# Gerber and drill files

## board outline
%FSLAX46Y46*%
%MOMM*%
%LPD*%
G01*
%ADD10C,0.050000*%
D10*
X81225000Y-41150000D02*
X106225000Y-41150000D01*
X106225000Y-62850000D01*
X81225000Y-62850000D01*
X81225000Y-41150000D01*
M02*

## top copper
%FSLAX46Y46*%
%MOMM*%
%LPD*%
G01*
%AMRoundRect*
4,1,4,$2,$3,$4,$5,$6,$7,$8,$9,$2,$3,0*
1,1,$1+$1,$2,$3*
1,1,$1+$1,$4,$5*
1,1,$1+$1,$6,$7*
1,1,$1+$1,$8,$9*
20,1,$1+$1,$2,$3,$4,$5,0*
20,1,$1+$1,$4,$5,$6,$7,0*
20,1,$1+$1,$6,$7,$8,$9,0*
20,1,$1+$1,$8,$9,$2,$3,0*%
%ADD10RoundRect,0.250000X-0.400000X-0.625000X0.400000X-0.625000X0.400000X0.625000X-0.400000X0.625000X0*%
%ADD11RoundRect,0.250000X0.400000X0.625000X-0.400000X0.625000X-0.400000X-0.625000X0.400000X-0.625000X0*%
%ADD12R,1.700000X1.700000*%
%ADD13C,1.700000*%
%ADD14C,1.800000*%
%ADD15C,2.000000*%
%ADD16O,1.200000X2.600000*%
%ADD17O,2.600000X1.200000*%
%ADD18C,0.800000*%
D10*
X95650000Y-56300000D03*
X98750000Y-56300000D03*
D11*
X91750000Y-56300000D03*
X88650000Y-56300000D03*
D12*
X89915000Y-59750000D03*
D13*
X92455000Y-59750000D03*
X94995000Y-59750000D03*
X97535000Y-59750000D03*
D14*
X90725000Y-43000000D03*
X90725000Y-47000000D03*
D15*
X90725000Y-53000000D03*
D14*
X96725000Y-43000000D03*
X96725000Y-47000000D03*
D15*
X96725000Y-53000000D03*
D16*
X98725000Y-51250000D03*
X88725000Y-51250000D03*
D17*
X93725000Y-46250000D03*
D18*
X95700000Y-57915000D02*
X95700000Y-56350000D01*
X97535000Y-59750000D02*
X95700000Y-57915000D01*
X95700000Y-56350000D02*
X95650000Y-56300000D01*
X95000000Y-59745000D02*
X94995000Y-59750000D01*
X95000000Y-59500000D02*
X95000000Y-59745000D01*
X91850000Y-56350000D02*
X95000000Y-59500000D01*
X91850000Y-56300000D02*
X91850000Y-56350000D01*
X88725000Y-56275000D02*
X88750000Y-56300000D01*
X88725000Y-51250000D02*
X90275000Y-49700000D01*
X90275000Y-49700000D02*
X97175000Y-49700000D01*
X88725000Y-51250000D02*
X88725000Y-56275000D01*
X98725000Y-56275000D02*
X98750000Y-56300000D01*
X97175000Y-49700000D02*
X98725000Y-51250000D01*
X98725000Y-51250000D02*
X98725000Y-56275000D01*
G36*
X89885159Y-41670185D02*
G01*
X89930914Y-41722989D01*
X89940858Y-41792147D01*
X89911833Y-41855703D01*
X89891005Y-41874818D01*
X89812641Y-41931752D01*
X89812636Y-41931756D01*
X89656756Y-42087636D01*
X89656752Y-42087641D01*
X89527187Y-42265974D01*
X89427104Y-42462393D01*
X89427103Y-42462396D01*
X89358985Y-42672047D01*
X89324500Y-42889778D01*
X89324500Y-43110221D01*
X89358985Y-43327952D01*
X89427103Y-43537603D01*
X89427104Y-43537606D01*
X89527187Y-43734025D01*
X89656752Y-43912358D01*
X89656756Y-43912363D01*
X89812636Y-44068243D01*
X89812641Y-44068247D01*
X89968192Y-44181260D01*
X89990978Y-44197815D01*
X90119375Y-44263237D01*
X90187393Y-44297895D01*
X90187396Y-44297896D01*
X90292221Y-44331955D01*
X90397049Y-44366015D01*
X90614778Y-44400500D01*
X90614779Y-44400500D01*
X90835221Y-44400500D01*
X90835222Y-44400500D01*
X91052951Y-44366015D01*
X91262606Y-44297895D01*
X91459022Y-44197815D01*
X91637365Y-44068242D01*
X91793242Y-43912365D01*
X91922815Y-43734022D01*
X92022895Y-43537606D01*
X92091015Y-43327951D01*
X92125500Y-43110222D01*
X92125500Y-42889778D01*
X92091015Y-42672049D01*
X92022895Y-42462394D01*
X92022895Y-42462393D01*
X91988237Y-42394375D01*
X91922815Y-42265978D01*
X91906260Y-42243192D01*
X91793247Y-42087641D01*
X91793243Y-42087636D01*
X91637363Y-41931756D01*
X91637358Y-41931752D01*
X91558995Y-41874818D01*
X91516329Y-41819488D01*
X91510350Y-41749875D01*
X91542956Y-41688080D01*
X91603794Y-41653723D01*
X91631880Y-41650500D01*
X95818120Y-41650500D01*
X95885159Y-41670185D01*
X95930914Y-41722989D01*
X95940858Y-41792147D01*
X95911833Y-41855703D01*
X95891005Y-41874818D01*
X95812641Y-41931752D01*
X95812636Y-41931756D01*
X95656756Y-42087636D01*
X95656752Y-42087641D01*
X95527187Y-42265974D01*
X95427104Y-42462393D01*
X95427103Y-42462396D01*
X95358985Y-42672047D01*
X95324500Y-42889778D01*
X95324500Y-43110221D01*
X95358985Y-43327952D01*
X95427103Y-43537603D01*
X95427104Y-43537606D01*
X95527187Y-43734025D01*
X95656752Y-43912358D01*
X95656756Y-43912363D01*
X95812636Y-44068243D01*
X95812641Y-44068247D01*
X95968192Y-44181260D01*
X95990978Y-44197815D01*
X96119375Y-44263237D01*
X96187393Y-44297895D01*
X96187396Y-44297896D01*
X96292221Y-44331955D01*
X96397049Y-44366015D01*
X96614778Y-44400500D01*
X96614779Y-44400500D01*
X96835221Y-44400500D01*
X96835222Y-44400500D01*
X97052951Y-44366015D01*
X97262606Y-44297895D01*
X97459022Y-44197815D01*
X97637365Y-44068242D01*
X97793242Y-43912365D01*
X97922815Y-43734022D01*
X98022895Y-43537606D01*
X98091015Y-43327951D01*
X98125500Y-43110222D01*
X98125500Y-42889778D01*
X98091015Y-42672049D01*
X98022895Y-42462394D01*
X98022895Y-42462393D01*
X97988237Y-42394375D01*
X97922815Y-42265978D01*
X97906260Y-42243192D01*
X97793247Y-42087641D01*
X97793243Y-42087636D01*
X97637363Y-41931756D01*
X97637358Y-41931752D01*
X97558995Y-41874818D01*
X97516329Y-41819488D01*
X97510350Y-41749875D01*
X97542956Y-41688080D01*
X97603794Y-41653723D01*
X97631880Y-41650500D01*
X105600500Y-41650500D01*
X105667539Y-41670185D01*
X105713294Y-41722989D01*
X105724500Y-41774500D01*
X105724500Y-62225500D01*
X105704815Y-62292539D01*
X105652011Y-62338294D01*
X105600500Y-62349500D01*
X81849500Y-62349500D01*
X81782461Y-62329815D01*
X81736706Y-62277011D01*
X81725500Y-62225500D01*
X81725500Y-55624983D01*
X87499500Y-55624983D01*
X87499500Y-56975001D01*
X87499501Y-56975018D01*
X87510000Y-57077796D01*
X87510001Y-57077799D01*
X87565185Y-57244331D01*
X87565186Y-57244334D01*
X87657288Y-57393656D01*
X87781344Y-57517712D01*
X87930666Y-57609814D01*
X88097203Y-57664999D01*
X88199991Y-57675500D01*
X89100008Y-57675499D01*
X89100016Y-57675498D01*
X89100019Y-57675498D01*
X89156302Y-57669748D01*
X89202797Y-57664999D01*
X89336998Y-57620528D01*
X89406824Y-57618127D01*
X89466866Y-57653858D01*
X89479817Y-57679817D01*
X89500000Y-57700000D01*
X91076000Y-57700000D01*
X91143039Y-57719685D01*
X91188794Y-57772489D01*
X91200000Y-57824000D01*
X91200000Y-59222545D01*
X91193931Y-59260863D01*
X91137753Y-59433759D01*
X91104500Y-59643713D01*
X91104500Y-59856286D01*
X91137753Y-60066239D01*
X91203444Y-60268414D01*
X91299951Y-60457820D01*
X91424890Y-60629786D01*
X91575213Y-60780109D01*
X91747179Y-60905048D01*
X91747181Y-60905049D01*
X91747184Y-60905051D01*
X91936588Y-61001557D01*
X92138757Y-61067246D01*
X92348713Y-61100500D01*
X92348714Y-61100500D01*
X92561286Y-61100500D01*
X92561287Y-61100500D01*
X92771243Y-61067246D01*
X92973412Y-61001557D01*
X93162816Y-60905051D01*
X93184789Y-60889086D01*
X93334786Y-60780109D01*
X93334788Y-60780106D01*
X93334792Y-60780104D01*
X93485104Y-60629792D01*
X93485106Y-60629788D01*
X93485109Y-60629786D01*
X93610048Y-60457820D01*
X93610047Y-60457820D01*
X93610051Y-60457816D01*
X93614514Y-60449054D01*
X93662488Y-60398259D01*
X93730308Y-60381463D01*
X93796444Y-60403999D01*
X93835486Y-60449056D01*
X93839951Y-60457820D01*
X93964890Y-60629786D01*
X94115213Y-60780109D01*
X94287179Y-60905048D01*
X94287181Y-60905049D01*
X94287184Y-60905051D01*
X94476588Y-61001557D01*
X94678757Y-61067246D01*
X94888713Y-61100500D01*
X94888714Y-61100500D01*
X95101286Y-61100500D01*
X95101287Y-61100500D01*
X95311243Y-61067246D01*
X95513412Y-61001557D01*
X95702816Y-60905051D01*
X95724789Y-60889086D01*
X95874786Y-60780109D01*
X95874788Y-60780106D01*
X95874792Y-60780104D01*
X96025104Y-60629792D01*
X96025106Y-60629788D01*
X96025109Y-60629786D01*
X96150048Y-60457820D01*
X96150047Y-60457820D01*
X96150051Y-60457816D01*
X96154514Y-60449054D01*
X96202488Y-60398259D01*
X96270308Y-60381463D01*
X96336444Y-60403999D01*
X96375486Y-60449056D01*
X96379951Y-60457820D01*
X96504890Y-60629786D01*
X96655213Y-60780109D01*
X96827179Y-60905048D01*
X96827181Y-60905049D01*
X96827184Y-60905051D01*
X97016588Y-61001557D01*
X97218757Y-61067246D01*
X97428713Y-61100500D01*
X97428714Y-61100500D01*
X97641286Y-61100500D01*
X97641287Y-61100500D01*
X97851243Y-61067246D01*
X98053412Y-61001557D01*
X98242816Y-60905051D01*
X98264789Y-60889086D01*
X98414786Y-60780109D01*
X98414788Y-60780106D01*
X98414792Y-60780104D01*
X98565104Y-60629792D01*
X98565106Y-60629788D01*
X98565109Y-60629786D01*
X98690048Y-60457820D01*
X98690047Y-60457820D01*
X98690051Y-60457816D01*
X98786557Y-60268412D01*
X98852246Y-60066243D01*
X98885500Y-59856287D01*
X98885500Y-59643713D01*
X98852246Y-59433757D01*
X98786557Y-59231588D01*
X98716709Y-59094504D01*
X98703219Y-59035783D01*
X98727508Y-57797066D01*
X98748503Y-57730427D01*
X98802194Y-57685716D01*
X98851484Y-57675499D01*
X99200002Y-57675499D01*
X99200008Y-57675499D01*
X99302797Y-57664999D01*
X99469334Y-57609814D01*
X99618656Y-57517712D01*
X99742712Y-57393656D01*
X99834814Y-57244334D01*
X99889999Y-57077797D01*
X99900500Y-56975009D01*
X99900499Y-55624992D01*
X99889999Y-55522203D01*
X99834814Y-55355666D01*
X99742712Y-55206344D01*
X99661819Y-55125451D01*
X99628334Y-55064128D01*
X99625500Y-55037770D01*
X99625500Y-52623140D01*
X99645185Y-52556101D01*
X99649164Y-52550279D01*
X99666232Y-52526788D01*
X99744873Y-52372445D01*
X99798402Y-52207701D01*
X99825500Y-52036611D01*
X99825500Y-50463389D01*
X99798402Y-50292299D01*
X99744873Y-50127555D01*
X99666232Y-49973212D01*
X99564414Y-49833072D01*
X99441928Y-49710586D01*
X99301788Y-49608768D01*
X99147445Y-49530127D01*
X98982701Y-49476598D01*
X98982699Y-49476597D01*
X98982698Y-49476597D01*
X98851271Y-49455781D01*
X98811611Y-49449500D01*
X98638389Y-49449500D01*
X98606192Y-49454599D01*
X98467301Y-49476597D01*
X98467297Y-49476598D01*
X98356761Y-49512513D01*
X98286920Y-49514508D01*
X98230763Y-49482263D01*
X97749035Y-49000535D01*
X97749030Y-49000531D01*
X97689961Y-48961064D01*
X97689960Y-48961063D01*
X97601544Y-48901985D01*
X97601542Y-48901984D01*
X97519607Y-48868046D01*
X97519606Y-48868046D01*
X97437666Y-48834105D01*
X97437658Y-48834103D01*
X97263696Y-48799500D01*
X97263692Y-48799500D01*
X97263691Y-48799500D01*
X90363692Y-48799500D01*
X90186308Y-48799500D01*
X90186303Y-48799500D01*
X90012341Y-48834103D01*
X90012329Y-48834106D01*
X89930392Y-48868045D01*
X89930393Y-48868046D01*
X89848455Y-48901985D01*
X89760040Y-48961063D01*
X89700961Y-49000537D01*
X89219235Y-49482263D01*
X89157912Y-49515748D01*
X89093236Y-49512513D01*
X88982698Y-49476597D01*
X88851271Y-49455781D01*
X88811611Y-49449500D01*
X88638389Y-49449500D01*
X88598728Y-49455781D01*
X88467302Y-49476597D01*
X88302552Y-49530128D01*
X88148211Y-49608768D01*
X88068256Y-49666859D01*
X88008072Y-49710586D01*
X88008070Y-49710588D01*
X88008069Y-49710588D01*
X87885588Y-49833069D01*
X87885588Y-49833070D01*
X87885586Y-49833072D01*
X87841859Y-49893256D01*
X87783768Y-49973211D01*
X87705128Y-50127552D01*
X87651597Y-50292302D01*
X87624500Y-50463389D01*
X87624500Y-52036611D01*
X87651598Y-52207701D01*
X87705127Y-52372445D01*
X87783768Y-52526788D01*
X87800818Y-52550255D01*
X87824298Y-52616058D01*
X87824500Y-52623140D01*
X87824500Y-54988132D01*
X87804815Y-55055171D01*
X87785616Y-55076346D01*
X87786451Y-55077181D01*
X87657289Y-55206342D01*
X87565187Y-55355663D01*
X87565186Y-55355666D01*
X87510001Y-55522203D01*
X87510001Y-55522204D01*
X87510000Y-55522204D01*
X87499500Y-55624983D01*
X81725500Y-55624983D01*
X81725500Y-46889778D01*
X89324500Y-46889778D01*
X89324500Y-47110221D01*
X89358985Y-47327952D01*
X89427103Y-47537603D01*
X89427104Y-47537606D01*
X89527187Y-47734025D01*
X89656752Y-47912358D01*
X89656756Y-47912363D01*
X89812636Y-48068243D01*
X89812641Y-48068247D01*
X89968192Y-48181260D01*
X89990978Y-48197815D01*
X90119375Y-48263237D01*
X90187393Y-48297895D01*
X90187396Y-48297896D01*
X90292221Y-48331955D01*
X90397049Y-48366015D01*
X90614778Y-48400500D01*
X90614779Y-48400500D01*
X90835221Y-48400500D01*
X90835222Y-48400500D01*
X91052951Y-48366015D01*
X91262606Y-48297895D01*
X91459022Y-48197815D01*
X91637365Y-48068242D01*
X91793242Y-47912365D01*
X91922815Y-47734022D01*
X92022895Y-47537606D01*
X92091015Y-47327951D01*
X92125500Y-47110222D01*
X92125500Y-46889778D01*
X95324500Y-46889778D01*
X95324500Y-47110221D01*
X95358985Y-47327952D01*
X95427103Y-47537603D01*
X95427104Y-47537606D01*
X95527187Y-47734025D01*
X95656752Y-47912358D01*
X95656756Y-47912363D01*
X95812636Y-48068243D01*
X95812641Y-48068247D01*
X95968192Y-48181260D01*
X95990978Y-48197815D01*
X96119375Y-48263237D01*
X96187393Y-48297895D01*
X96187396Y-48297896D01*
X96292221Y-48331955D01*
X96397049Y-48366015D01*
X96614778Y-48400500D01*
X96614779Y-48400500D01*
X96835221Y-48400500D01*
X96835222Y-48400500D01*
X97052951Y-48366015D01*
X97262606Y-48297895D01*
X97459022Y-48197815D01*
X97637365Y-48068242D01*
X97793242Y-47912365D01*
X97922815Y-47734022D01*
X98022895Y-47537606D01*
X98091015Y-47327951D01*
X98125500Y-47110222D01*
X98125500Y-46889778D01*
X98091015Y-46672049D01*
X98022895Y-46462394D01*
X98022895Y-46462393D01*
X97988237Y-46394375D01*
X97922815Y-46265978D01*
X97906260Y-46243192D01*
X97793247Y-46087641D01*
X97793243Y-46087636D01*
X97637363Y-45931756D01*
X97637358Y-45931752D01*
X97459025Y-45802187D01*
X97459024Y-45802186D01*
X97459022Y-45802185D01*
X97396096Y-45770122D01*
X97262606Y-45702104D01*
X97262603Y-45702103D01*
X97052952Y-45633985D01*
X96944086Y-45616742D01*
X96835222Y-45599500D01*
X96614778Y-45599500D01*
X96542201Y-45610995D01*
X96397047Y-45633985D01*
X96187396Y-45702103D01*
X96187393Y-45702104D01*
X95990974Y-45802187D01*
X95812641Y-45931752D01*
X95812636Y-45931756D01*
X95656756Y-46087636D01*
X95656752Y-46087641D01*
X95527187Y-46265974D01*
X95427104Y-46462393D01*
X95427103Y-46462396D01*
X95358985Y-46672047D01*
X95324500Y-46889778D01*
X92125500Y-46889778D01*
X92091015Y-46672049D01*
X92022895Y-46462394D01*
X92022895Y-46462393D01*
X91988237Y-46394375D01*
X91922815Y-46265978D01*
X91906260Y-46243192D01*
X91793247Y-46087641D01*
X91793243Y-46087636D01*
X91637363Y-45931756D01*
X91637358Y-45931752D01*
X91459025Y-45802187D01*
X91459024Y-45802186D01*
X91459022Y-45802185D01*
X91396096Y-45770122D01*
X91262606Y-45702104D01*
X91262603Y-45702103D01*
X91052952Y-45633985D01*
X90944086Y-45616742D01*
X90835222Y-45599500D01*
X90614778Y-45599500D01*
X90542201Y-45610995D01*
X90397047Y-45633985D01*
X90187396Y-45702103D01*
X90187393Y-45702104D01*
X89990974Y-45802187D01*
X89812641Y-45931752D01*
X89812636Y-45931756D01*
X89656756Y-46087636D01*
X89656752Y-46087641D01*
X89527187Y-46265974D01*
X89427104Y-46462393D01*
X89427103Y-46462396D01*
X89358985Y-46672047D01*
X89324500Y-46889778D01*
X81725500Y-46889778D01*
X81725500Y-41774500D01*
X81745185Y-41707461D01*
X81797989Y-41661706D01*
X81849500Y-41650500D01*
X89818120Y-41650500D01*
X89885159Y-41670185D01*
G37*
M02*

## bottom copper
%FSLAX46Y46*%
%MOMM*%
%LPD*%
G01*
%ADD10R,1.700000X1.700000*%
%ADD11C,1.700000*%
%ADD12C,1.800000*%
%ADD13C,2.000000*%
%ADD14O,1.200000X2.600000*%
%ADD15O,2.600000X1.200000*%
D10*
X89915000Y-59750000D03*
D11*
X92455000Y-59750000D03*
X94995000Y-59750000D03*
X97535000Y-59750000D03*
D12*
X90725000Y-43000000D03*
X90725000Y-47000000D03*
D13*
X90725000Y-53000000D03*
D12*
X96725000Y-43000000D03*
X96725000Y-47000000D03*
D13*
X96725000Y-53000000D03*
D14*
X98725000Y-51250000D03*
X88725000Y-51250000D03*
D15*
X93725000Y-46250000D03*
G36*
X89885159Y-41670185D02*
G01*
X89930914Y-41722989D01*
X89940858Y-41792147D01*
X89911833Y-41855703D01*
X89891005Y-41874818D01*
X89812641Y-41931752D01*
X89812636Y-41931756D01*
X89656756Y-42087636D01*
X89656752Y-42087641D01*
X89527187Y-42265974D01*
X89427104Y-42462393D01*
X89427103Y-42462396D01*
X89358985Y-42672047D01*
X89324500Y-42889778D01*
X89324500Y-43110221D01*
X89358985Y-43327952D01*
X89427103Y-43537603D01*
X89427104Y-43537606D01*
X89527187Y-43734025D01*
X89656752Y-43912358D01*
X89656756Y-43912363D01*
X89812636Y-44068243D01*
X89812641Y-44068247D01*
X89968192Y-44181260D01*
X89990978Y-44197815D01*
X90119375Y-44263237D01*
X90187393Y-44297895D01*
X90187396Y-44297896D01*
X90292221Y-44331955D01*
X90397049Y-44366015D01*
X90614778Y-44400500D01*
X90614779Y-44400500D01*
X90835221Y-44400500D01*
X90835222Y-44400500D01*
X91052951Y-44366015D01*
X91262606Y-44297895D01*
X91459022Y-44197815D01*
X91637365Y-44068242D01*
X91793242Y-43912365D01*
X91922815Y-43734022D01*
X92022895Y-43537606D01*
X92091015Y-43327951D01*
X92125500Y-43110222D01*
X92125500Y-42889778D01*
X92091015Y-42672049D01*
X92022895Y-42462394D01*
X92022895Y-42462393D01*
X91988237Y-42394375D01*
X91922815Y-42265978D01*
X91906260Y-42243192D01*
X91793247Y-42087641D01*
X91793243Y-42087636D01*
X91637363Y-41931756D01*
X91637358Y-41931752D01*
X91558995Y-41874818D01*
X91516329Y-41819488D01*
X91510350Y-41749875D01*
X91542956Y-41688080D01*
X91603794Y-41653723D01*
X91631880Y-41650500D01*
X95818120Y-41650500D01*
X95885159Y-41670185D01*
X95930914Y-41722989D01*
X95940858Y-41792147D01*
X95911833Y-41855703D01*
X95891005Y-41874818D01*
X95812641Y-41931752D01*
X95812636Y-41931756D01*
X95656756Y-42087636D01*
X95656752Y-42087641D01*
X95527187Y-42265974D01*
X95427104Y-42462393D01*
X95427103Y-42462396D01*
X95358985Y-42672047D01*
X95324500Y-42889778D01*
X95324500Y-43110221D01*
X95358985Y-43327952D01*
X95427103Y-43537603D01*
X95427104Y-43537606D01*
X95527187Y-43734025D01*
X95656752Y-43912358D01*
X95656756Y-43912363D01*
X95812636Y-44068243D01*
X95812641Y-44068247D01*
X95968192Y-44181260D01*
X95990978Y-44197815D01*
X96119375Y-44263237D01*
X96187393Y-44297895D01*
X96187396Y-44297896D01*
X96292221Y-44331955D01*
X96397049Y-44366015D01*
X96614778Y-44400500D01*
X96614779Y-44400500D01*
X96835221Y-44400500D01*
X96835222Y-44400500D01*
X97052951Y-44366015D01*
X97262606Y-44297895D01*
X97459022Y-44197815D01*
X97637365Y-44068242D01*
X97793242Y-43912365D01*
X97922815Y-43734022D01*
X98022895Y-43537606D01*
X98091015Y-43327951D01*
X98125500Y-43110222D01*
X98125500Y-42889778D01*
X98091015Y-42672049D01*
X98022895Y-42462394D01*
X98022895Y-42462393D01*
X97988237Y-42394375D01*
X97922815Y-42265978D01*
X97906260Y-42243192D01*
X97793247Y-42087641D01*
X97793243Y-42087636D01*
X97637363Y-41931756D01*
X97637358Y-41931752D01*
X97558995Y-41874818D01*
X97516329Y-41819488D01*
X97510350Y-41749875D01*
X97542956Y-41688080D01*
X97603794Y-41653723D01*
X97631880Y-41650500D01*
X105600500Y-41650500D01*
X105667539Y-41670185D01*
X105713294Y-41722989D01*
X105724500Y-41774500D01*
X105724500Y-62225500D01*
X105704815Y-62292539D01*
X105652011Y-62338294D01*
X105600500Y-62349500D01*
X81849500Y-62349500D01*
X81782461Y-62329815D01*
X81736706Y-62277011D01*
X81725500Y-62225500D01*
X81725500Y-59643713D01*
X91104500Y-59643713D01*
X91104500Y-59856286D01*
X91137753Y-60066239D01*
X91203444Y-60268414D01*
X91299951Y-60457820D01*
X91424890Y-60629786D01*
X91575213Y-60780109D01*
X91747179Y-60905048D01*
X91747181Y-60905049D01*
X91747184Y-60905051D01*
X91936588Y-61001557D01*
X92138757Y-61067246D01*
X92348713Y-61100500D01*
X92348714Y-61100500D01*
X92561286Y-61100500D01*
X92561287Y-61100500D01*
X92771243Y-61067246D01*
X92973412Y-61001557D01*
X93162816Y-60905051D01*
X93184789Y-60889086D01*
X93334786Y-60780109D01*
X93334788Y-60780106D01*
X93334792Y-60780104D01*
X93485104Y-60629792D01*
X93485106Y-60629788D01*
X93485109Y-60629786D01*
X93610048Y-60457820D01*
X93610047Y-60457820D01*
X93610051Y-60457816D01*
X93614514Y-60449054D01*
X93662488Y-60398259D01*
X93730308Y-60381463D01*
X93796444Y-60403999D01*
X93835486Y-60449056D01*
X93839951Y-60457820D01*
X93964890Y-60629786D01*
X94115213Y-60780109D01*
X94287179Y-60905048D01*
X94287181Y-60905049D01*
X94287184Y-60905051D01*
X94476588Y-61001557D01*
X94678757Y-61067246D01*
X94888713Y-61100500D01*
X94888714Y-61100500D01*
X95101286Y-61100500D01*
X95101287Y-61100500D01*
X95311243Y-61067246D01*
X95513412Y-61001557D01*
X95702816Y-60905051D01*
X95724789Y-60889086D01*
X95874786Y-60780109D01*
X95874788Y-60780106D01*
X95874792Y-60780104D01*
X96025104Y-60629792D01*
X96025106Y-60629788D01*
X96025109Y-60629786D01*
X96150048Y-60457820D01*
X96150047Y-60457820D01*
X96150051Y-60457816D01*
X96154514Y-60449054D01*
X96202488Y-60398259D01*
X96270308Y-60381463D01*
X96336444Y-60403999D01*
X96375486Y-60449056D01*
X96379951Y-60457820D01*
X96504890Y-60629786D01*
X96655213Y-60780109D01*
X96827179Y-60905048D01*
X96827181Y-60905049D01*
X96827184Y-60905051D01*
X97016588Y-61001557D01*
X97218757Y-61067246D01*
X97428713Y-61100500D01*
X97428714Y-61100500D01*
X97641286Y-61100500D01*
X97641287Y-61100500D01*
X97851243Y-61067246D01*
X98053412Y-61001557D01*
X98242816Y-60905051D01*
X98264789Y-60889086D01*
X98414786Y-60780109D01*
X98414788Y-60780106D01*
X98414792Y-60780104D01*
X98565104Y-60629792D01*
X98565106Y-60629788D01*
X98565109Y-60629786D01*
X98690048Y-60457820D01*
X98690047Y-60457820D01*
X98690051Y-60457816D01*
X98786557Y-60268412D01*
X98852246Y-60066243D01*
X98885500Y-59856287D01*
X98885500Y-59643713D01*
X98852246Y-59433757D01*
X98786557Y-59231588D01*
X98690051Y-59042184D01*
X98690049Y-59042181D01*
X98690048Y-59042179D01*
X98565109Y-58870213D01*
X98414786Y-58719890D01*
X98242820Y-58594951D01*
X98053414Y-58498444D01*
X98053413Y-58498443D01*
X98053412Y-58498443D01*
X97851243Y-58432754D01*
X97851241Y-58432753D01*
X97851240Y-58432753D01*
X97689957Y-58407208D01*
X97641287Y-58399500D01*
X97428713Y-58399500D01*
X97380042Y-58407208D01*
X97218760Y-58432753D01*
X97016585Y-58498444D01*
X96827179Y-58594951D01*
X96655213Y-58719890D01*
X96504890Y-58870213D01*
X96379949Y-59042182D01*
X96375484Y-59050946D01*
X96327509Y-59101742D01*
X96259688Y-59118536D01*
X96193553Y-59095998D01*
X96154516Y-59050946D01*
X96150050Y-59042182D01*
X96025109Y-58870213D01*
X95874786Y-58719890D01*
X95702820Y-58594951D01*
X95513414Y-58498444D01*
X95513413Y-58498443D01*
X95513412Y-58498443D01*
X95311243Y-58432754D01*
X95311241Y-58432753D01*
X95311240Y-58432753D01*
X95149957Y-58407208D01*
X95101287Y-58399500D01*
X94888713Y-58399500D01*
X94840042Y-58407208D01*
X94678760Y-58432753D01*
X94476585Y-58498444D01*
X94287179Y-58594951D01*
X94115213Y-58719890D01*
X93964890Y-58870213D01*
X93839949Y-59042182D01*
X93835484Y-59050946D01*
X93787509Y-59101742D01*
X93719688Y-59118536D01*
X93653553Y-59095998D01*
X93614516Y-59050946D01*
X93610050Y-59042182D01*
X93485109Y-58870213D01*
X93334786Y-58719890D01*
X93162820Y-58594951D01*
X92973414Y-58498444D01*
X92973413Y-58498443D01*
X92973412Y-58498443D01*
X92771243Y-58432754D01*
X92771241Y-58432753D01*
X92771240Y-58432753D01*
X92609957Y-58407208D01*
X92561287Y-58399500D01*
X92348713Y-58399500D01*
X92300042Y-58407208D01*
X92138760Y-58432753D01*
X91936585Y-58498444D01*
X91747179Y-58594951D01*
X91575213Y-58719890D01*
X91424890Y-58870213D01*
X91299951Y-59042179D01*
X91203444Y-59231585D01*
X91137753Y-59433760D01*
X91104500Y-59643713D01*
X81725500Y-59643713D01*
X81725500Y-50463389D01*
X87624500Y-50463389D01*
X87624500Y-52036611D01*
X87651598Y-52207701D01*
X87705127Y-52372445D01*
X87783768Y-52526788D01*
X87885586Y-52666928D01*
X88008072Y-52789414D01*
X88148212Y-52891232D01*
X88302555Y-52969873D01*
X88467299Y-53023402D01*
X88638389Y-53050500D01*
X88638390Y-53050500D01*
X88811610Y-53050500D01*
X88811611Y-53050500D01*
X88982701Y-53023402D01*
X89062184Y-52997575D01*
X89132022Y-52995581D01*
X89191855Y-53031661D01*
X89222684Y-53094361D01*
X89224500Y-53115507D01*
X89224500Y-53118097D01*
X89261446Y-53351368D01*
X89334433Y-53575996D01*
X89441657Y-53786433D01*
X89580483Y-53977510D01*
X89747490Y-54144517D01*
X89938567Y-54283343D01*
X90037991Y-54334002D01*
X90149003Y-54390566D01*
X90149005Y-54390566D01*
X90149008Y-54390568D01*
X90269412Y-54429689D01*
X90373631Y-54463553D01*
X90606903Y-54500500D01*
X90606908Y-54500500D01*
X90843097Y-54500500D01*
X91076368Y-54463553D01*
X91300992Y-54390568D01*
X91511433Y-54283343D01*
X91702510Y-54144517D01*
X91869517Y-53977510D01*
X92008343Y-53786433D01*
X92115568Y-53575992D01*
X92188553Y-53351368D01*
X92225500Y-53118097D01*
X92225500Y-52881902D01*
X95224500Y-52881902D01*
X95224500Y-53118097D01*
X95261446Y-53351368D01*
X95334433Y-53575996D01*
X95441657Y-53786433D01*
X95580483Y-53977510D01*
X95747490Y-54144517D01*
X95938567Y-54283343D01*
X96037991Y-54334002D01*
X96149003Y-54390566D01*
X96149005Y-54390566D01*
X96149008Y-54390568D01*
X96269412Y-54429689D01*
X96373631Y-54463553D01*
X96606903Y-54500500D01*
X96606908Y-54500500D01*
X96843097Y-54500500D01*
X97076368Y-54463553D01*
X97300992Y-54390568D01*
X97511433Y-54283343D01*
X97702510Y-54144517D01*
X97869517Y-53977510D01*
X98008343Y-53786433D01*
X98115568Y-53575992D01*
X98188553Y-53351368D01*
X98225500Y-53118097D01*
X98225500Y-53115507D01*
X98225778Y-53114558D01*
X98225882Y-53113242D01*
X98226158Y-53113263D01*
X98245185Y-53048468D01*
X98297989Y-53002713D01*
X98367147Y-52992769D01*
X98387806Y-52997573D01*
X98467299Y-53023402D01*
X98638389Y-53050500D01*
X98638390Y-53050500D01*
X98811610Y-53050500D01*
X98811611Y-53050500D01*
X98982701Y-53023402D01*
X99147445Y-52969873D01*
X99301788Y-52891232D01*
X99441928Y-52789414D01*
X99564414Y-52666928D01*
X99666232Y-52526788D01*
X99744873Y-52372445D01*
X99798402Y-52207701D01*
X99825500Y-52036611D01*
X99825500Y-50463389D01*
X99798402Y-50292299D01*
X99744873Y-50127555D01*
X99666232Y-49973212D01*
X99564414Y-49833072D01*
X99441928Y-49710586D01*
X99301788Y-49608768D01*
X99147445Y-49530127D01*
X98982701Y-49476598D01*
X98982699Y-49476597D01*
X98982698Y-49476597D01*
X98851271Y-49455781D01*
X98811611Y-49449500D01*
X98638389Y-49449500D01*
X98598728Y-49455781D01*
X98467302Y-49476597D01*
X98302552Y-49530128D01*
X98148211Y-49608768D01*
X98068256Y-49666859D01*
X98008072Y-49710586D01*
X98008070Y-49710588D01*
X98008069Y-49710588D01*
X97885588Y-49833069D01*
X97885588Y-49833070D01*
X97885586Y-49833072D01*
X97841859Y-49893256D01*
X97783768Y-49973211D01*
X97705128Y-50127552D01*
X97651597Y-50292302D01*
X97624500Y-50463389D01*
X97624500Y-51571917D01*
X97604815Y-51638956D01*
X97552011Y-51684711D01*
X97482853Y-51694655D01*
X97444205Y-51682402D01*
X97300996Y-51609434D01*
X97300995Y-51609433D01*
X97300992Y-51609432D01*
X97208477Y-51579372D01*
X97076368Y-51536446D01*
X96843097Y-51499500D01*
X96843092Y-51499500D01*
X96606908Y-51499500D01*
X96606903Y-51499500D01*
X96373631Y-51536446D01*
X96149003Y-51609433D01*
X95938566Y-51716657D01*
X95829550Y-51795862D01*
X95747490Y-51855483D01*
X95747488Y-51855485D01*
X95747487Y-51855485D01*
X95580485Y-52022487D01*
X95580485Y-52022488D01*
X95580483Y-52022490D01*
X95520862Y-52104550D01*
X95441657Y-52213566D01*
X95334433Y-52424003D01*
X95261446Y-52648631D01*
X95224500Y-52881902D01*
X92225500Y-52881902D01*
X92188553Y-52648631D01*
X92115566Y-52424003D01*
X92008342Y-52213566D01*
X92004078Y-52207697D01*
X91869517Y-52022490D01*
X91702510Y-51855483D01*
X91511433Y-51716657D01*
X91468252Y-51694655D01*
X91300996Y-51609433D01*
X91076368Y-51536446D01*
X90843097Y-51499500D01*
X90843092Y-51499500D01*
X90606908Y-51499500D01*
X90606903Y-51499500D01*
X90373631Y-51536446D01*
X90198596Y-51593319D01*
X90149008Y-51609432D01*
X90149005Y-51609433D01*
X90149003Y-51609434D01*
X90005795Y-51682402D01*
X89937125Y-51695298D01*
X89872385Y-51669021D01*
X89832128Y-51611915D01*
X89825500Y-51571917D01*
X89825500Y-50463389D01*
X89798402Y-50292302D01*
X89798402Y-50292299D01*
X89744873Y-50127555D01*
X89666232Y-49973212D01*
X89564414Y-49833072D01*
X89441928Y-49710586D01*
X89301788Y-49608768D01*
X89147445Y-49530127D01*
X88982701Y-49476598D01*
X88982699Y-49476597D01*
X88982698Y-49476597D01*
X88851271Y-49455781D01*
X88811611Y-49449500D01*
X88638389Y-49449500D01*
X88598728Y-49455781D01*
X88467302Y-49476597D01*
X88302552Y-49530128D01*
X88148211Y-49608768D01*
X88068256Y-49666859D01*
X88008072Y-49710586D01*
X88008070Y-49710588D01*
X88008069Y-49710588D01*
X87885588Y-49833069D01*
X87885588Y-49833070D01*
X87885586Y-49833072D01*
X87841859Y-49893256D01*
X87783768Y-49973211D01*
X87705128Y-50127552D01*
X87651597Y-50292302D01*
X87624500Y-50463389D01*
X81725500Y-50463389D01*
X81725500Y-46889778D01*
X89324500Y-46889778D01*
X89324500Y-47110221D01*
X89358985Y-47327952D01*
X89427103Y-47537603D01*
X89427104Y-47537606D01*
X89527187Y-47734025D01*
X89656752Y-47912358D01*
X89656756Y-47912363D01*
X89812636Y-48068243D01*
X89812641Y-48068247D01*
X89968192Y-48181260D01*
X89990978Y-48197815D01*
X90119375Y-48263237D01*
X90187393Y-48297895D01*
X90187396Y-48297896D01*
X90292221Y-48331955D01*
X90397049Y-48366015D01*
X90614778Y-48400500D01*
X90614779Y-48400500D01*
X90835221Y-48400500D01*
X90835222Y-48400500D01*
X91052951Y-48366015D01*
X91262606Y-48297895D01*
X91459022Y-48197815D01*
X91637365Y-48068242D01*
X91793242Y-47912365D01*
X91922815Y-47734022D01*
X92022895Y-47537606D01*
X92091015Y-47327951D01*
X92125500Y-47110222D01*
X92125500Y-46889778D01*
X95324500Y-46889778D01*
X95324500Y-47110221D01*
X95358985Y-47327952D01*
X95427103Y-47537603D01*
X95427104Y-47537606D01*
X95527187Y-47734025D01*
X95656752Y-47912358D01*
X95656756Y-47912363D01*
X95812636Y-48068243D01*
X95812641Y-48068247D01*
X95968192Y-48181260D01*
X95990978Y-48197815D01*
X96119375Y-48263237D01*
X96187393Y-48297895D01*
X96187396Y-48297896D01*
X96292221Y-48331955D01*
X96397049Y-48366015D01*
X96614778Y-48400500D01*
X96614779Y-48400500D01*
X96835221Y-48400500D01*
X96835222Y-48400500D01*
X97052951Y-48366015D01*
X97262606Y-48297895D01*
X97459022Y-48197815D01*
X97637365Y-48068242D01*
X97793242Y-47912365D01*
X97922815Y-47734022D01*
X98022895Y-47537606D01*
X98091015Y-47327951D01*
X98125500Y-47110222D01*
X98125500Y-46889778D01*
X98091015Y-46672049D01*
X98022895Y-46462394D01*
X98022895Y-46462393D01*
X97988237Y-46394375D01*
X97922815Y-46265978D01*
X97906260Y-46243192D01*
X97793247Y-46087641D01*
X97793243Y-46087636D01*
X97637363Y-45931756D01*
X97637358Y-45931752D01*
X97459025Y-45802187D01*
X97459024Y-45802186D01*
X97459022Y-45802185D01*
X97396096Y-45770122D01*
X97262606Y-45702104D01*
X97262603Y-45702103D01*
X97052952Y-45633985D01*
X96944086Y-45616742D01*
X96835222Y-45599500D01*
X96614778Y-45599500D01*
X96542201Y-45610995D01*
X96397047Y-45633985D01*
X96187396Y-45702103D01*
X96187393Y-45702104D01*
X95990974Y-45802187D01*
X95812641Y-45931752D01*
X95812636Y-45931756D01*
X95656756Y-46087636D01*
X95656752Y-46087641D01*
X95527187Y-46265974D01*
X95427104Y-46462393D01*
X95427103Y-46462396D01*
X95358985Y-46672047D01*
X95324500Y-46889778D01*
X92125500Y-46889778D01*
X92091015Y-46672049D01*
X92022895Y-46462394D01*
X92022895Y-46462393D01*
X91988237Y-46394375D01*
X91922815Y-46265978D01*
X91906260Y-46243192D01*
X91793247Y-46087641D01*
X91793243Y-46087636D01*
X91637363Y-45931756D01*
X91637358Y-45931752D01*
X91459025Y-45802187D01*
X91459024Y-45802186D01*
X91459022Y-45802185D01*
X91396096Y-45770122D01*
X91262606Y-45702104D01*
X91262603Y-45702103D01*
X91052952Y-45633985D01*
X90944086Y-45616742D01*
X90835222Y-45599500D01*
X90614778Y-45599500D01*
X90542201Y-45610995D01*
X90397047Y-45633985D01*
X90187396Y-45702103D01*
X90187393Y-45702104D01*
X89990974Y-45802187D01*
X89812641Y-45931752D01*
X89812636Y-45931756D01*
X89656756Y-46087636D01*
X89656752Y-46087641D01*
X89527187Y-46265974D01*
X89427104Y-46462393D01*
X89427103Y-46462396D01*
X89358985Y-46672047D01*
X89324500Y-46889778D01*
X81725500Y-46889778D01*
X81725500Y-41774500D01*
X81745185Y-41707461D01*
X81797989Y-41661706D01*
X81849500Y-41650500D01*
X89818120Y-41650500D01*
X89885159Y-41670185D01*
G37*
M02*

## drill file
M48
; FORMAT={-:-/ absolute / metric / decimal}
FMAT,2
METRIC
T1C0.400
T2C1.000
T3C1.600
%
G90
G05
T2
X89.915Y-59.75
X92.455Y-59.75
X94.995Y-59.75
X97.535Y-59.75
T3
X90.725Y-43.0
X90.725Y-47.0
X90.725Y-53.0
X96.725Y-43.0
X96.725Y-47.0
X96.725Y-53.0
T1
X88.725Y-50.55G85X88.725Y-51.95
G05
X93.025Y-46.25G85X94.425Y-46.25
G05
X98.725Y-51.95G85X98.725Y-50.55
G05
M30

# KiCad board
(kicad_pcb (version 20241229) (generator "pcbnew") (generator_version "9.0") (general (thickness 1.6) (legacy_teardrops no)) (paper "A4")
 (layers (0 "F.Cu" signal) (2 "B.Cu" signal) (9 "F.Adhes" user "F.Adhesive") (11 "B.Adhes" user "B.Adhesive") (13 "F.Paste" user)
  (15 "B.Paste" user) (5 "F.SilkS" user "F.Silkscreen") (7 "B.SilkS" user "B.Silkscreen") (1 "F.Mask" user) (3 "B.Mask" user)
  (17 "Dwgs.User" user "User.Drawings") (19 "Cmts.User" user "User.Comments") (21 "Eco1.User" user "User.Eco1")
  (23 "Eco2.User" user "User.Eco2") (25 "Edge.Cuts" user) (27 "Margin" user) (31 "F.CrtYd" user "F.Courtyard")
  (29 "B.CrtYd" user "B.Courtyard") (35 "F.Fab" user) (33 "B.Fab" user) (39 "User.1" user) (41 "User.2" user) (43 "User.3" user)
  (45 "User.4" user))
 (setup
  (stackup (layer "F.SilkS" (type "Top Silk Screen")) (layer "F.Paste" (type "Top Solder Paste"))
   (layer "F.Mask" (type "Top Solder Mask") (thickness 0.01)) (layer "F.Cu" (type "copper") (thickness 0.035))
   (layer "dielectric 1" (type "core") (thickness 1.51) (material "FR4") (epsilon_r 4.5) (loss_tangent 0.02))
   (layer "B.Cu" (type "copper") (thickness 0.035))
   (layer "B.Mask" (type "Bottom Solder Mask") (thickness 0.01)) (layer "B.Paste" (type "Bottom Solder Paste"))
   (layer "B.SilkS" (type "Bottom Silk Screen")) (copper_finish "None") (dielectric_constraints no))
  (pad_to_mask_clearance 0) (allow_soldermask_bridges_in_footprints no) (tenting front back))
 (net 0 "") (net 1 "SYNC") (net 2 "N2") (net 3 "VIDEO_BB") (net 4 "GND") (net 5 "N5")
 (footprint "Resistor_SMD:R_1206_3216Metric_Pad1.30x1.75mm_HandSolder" (layer "F.Cu") (at 97.2 56.3)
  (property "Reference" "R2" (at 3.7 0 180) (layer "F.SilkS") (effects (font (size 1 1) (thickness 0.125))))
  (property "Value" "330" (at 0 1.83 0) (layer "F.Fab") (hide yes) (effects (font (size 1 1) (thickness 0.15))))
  (pad "1" smd roundrect (at -1.55 0) (size 1.3 1.75) (layers "F.Cu" "F.Mask" "F.Paste") (roundrect_rratio 0.192308) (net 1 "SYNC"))
  (pad "2" smd roundrect (at 1.55 0) (size 1.3 1.75) (layers "F.Cu" "F.Mask" "F.Paste") (roundrect_rratio 0.192308) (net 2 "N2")))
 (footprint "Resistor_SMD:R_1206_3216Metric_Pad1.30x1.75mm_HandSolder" (layer "F.Cu") (at 90.2 56.3 180)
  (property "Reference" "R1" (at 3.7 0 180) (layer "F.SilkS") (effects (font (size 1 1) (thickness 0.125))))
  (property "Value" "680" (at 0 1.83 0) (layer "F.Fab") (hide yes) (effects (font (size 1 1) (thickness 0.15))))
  (pad "1" smd roundrect (at -1.55 0 180) (size 1.3 1.75) (layers "F.Cu" "F.Mask" "F.Paste") (roundrect_rratio 0.192308) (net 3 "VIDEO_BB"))
  (pad "2" smd roundrect (at 1.55 0 180) (size 1.3 1.75) (layers "F.Cu" "F.Mask" "F.Paste") (roundrect_rratio 0.192308) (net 2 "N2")))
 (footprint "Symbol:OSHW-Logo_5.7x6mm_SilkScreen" (layer "F.Cu") (at 101.97 45.31 -90)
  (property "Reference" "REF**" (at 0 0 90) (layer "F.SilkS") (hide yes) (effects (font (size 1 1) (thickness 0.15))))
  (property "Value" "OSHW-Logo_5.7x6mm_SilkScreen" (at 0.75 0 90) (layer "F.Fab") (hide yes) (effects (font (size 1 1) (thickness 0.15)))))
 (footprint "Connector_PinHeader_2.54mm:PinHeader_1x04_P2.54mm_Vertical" (layer "F.Cu") (at 89.915 59.75 90)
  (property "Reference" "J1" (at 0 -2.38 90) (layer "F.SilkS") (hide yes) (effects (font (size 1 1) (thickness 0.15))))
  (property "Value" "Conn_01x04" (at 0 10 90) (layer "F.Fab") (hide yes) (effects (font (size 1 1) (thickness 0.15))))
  (pad "1" thru_hole rect (at 0 0 90) (size 1.7 1.7) (drill 1) (layers "*.Cu" "*.Mask") (remove_unused_layers no) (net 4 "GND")
   (zone_connect 2))
  (pad "2" thru_hole circle (at 0 2.54 90) (size 1.7 1.7) (drill 1) (layers "*.Cu" "*.Mask") (remove_unused_layers no) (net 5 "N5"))
  (pad "3" thru_hole circle (at 0 5.08 90) (size 1.7 1.7) (drill 1) (layers "*.Cu" "*.Mask") (remove_unused_layers no) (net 3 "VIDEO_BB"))
  (pad "4" thru_hole circle (at 0 7.62 90) (size 1.7 1.7) (drill 1) (layers "*.Cu" "*.Mask") (remove_unused_layers no) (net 1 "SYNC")))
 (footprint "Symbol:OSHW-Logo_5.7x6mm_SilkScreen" (layer "B.Cu") (at 103.54 45.33 -90)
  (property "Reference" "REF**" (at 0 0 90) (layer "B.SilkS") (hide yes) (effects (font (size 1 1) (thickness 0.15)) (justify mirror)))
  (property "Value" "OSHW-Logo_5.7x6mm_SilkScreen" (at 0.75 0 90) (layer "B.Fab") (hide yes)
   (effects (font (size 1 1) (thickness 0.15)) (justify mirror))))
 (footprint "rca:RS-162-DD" (layer "B.Cu") (at 93.725 45)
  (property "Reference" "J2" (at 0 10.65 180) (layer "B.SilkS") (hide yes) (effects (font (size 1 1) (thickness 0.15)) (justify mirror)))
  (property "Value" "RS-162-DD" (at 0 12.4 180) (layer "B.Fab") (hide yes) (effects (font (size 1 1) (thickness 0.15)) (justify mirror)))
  (pad "" np_thru_hole circle (at -3 -2) (size 1.8 1.8) (drill 1.6) (layers "*.Cu" "*.Mask"))
  (pad "" np_thru_hole circle (at -3 2) (size 1.8 1.8) (drill 1.6) (layers "*.Cu" "*.Mask"))
  (pad "" np_thru_hole circle (at -3 8) (size 2 2) (drill 1.6) (layers "*.Cu" "*.Mask"))
  (pad "" np_thru_hole circle (at 3 -2) (size 1.8 1.8) (drill 1.6) (layers "*.Cu" "*.Mask"))
  (pad "" np_thru_hole circle (at 3 2) (size 1.8 1.8) (drill 1.6) (layers "*.Cu" "*.Mask"))
  (pad "" np_thru_hole circle (at 3 8) (size 2 2) (drill 1.6) (layers "*.Cu" "*.Mask"))
  (pad "2" thru_hole oval (at 5 6.25 180) (size 1.2 2.6) (drill oval 0.4 1.8) (layers "*.Cu" "*.Mask") (remove_unused_layers no)
   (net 2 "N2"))
  (pad "3" thru_hole oval (at -5 6.25) (size 1.2 2.6) (drill oval 0.4 1.8) (layers "*.Cu" "*.Mask") (remove_unused_layers no) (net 2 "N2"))
  (pad "4" thru_hole oval (at 0 1.25) (size 2.6 1.2) (drill oval 1.8 0.4) (layers "*.Cu" "*.Mask") (remove_unused_layers no) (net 4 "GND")
   (zone_connect 2)))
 (gr_rect (start 81.225 41.15) (end 106.225 62.85) (stroke (width 0.05) (type solid)) (fill no) (layer "Edge.Cuts"))
 (segment (start 95.7 57.915) (end 95.7 56.35) (width 0.8) (layer "F.Cu") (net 1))
 (segment (start 97.535 59.75) (end 95.7 57.915) (width 0.8) (layer "F.Cu") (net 1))
 (segment (start 95.7 56.35) (end 95.65 56.3) (width 0.8) (layer "F.Cu") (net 1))
 (segment (start 95 59.745) (end 94.995 59.75) (width 0.8) (layer "F.Cu") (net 3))
 (segment (start 95 59.5) (end 95 59.745) (width 0.8) (layer "F.Cu") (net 3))
 (segment (start 91.85 56.35) (end 95 59.5) (width 0.8) (layer "F.Cu") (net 3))
 (segment (start 91.85 56.3) (end 91.85 56.35) (width 0.8) (layer "F.Cu") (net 3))
 (segment (start 88.725 56.275) (end 88.75 56.3) (width 0.8) (layer "F.Cu") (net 2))
 (segment (start 88.725 51.25) (end 90.275 49.7) (width 0.8) (layer "F.Cu") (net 2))
 (segment (start 90.275 49.7) (end 97.175 49.7) (width 0.8) (layer "F.Cu") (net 2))
 (segment (start 88.725 51.25) (end 88.725 56.275) (width 0.8) (layer "F.Cu") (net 2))
 (segment (start 98.725 56.275) (end 98.75 56.3) (width 0.8) (layer "F.Cu") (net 2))
 (segment (start 97.175 49.7) (end 98.725 51.25) (width 0.8) (layer "F.Cu") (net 2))
 (segment (start 98.725 51.25) (end 98.725 56.275) (width 0.8) (layer "F.Cu") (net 2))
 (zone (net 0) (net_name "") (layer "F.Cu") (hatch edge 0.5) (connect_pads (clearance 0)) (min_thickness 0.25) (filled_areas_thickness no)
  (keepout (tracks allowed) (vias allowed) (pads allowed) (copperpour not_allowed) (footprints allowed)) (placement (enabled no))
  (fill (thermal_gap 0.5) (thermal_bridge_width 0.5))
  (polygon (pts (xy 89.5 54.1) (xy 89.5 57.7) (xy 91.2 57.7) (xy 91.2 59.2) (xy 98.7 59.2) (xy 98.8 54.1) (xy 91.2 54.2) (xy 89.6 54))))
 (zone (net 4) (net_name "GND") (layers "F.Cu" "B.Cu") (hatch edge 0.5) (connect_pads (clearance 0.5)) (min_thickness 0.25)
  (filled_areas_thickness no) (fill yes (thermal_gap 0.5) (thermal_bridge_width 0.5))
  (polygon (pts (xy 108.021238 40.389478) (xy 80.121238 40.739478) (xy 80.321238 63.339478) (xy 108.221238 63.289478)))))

